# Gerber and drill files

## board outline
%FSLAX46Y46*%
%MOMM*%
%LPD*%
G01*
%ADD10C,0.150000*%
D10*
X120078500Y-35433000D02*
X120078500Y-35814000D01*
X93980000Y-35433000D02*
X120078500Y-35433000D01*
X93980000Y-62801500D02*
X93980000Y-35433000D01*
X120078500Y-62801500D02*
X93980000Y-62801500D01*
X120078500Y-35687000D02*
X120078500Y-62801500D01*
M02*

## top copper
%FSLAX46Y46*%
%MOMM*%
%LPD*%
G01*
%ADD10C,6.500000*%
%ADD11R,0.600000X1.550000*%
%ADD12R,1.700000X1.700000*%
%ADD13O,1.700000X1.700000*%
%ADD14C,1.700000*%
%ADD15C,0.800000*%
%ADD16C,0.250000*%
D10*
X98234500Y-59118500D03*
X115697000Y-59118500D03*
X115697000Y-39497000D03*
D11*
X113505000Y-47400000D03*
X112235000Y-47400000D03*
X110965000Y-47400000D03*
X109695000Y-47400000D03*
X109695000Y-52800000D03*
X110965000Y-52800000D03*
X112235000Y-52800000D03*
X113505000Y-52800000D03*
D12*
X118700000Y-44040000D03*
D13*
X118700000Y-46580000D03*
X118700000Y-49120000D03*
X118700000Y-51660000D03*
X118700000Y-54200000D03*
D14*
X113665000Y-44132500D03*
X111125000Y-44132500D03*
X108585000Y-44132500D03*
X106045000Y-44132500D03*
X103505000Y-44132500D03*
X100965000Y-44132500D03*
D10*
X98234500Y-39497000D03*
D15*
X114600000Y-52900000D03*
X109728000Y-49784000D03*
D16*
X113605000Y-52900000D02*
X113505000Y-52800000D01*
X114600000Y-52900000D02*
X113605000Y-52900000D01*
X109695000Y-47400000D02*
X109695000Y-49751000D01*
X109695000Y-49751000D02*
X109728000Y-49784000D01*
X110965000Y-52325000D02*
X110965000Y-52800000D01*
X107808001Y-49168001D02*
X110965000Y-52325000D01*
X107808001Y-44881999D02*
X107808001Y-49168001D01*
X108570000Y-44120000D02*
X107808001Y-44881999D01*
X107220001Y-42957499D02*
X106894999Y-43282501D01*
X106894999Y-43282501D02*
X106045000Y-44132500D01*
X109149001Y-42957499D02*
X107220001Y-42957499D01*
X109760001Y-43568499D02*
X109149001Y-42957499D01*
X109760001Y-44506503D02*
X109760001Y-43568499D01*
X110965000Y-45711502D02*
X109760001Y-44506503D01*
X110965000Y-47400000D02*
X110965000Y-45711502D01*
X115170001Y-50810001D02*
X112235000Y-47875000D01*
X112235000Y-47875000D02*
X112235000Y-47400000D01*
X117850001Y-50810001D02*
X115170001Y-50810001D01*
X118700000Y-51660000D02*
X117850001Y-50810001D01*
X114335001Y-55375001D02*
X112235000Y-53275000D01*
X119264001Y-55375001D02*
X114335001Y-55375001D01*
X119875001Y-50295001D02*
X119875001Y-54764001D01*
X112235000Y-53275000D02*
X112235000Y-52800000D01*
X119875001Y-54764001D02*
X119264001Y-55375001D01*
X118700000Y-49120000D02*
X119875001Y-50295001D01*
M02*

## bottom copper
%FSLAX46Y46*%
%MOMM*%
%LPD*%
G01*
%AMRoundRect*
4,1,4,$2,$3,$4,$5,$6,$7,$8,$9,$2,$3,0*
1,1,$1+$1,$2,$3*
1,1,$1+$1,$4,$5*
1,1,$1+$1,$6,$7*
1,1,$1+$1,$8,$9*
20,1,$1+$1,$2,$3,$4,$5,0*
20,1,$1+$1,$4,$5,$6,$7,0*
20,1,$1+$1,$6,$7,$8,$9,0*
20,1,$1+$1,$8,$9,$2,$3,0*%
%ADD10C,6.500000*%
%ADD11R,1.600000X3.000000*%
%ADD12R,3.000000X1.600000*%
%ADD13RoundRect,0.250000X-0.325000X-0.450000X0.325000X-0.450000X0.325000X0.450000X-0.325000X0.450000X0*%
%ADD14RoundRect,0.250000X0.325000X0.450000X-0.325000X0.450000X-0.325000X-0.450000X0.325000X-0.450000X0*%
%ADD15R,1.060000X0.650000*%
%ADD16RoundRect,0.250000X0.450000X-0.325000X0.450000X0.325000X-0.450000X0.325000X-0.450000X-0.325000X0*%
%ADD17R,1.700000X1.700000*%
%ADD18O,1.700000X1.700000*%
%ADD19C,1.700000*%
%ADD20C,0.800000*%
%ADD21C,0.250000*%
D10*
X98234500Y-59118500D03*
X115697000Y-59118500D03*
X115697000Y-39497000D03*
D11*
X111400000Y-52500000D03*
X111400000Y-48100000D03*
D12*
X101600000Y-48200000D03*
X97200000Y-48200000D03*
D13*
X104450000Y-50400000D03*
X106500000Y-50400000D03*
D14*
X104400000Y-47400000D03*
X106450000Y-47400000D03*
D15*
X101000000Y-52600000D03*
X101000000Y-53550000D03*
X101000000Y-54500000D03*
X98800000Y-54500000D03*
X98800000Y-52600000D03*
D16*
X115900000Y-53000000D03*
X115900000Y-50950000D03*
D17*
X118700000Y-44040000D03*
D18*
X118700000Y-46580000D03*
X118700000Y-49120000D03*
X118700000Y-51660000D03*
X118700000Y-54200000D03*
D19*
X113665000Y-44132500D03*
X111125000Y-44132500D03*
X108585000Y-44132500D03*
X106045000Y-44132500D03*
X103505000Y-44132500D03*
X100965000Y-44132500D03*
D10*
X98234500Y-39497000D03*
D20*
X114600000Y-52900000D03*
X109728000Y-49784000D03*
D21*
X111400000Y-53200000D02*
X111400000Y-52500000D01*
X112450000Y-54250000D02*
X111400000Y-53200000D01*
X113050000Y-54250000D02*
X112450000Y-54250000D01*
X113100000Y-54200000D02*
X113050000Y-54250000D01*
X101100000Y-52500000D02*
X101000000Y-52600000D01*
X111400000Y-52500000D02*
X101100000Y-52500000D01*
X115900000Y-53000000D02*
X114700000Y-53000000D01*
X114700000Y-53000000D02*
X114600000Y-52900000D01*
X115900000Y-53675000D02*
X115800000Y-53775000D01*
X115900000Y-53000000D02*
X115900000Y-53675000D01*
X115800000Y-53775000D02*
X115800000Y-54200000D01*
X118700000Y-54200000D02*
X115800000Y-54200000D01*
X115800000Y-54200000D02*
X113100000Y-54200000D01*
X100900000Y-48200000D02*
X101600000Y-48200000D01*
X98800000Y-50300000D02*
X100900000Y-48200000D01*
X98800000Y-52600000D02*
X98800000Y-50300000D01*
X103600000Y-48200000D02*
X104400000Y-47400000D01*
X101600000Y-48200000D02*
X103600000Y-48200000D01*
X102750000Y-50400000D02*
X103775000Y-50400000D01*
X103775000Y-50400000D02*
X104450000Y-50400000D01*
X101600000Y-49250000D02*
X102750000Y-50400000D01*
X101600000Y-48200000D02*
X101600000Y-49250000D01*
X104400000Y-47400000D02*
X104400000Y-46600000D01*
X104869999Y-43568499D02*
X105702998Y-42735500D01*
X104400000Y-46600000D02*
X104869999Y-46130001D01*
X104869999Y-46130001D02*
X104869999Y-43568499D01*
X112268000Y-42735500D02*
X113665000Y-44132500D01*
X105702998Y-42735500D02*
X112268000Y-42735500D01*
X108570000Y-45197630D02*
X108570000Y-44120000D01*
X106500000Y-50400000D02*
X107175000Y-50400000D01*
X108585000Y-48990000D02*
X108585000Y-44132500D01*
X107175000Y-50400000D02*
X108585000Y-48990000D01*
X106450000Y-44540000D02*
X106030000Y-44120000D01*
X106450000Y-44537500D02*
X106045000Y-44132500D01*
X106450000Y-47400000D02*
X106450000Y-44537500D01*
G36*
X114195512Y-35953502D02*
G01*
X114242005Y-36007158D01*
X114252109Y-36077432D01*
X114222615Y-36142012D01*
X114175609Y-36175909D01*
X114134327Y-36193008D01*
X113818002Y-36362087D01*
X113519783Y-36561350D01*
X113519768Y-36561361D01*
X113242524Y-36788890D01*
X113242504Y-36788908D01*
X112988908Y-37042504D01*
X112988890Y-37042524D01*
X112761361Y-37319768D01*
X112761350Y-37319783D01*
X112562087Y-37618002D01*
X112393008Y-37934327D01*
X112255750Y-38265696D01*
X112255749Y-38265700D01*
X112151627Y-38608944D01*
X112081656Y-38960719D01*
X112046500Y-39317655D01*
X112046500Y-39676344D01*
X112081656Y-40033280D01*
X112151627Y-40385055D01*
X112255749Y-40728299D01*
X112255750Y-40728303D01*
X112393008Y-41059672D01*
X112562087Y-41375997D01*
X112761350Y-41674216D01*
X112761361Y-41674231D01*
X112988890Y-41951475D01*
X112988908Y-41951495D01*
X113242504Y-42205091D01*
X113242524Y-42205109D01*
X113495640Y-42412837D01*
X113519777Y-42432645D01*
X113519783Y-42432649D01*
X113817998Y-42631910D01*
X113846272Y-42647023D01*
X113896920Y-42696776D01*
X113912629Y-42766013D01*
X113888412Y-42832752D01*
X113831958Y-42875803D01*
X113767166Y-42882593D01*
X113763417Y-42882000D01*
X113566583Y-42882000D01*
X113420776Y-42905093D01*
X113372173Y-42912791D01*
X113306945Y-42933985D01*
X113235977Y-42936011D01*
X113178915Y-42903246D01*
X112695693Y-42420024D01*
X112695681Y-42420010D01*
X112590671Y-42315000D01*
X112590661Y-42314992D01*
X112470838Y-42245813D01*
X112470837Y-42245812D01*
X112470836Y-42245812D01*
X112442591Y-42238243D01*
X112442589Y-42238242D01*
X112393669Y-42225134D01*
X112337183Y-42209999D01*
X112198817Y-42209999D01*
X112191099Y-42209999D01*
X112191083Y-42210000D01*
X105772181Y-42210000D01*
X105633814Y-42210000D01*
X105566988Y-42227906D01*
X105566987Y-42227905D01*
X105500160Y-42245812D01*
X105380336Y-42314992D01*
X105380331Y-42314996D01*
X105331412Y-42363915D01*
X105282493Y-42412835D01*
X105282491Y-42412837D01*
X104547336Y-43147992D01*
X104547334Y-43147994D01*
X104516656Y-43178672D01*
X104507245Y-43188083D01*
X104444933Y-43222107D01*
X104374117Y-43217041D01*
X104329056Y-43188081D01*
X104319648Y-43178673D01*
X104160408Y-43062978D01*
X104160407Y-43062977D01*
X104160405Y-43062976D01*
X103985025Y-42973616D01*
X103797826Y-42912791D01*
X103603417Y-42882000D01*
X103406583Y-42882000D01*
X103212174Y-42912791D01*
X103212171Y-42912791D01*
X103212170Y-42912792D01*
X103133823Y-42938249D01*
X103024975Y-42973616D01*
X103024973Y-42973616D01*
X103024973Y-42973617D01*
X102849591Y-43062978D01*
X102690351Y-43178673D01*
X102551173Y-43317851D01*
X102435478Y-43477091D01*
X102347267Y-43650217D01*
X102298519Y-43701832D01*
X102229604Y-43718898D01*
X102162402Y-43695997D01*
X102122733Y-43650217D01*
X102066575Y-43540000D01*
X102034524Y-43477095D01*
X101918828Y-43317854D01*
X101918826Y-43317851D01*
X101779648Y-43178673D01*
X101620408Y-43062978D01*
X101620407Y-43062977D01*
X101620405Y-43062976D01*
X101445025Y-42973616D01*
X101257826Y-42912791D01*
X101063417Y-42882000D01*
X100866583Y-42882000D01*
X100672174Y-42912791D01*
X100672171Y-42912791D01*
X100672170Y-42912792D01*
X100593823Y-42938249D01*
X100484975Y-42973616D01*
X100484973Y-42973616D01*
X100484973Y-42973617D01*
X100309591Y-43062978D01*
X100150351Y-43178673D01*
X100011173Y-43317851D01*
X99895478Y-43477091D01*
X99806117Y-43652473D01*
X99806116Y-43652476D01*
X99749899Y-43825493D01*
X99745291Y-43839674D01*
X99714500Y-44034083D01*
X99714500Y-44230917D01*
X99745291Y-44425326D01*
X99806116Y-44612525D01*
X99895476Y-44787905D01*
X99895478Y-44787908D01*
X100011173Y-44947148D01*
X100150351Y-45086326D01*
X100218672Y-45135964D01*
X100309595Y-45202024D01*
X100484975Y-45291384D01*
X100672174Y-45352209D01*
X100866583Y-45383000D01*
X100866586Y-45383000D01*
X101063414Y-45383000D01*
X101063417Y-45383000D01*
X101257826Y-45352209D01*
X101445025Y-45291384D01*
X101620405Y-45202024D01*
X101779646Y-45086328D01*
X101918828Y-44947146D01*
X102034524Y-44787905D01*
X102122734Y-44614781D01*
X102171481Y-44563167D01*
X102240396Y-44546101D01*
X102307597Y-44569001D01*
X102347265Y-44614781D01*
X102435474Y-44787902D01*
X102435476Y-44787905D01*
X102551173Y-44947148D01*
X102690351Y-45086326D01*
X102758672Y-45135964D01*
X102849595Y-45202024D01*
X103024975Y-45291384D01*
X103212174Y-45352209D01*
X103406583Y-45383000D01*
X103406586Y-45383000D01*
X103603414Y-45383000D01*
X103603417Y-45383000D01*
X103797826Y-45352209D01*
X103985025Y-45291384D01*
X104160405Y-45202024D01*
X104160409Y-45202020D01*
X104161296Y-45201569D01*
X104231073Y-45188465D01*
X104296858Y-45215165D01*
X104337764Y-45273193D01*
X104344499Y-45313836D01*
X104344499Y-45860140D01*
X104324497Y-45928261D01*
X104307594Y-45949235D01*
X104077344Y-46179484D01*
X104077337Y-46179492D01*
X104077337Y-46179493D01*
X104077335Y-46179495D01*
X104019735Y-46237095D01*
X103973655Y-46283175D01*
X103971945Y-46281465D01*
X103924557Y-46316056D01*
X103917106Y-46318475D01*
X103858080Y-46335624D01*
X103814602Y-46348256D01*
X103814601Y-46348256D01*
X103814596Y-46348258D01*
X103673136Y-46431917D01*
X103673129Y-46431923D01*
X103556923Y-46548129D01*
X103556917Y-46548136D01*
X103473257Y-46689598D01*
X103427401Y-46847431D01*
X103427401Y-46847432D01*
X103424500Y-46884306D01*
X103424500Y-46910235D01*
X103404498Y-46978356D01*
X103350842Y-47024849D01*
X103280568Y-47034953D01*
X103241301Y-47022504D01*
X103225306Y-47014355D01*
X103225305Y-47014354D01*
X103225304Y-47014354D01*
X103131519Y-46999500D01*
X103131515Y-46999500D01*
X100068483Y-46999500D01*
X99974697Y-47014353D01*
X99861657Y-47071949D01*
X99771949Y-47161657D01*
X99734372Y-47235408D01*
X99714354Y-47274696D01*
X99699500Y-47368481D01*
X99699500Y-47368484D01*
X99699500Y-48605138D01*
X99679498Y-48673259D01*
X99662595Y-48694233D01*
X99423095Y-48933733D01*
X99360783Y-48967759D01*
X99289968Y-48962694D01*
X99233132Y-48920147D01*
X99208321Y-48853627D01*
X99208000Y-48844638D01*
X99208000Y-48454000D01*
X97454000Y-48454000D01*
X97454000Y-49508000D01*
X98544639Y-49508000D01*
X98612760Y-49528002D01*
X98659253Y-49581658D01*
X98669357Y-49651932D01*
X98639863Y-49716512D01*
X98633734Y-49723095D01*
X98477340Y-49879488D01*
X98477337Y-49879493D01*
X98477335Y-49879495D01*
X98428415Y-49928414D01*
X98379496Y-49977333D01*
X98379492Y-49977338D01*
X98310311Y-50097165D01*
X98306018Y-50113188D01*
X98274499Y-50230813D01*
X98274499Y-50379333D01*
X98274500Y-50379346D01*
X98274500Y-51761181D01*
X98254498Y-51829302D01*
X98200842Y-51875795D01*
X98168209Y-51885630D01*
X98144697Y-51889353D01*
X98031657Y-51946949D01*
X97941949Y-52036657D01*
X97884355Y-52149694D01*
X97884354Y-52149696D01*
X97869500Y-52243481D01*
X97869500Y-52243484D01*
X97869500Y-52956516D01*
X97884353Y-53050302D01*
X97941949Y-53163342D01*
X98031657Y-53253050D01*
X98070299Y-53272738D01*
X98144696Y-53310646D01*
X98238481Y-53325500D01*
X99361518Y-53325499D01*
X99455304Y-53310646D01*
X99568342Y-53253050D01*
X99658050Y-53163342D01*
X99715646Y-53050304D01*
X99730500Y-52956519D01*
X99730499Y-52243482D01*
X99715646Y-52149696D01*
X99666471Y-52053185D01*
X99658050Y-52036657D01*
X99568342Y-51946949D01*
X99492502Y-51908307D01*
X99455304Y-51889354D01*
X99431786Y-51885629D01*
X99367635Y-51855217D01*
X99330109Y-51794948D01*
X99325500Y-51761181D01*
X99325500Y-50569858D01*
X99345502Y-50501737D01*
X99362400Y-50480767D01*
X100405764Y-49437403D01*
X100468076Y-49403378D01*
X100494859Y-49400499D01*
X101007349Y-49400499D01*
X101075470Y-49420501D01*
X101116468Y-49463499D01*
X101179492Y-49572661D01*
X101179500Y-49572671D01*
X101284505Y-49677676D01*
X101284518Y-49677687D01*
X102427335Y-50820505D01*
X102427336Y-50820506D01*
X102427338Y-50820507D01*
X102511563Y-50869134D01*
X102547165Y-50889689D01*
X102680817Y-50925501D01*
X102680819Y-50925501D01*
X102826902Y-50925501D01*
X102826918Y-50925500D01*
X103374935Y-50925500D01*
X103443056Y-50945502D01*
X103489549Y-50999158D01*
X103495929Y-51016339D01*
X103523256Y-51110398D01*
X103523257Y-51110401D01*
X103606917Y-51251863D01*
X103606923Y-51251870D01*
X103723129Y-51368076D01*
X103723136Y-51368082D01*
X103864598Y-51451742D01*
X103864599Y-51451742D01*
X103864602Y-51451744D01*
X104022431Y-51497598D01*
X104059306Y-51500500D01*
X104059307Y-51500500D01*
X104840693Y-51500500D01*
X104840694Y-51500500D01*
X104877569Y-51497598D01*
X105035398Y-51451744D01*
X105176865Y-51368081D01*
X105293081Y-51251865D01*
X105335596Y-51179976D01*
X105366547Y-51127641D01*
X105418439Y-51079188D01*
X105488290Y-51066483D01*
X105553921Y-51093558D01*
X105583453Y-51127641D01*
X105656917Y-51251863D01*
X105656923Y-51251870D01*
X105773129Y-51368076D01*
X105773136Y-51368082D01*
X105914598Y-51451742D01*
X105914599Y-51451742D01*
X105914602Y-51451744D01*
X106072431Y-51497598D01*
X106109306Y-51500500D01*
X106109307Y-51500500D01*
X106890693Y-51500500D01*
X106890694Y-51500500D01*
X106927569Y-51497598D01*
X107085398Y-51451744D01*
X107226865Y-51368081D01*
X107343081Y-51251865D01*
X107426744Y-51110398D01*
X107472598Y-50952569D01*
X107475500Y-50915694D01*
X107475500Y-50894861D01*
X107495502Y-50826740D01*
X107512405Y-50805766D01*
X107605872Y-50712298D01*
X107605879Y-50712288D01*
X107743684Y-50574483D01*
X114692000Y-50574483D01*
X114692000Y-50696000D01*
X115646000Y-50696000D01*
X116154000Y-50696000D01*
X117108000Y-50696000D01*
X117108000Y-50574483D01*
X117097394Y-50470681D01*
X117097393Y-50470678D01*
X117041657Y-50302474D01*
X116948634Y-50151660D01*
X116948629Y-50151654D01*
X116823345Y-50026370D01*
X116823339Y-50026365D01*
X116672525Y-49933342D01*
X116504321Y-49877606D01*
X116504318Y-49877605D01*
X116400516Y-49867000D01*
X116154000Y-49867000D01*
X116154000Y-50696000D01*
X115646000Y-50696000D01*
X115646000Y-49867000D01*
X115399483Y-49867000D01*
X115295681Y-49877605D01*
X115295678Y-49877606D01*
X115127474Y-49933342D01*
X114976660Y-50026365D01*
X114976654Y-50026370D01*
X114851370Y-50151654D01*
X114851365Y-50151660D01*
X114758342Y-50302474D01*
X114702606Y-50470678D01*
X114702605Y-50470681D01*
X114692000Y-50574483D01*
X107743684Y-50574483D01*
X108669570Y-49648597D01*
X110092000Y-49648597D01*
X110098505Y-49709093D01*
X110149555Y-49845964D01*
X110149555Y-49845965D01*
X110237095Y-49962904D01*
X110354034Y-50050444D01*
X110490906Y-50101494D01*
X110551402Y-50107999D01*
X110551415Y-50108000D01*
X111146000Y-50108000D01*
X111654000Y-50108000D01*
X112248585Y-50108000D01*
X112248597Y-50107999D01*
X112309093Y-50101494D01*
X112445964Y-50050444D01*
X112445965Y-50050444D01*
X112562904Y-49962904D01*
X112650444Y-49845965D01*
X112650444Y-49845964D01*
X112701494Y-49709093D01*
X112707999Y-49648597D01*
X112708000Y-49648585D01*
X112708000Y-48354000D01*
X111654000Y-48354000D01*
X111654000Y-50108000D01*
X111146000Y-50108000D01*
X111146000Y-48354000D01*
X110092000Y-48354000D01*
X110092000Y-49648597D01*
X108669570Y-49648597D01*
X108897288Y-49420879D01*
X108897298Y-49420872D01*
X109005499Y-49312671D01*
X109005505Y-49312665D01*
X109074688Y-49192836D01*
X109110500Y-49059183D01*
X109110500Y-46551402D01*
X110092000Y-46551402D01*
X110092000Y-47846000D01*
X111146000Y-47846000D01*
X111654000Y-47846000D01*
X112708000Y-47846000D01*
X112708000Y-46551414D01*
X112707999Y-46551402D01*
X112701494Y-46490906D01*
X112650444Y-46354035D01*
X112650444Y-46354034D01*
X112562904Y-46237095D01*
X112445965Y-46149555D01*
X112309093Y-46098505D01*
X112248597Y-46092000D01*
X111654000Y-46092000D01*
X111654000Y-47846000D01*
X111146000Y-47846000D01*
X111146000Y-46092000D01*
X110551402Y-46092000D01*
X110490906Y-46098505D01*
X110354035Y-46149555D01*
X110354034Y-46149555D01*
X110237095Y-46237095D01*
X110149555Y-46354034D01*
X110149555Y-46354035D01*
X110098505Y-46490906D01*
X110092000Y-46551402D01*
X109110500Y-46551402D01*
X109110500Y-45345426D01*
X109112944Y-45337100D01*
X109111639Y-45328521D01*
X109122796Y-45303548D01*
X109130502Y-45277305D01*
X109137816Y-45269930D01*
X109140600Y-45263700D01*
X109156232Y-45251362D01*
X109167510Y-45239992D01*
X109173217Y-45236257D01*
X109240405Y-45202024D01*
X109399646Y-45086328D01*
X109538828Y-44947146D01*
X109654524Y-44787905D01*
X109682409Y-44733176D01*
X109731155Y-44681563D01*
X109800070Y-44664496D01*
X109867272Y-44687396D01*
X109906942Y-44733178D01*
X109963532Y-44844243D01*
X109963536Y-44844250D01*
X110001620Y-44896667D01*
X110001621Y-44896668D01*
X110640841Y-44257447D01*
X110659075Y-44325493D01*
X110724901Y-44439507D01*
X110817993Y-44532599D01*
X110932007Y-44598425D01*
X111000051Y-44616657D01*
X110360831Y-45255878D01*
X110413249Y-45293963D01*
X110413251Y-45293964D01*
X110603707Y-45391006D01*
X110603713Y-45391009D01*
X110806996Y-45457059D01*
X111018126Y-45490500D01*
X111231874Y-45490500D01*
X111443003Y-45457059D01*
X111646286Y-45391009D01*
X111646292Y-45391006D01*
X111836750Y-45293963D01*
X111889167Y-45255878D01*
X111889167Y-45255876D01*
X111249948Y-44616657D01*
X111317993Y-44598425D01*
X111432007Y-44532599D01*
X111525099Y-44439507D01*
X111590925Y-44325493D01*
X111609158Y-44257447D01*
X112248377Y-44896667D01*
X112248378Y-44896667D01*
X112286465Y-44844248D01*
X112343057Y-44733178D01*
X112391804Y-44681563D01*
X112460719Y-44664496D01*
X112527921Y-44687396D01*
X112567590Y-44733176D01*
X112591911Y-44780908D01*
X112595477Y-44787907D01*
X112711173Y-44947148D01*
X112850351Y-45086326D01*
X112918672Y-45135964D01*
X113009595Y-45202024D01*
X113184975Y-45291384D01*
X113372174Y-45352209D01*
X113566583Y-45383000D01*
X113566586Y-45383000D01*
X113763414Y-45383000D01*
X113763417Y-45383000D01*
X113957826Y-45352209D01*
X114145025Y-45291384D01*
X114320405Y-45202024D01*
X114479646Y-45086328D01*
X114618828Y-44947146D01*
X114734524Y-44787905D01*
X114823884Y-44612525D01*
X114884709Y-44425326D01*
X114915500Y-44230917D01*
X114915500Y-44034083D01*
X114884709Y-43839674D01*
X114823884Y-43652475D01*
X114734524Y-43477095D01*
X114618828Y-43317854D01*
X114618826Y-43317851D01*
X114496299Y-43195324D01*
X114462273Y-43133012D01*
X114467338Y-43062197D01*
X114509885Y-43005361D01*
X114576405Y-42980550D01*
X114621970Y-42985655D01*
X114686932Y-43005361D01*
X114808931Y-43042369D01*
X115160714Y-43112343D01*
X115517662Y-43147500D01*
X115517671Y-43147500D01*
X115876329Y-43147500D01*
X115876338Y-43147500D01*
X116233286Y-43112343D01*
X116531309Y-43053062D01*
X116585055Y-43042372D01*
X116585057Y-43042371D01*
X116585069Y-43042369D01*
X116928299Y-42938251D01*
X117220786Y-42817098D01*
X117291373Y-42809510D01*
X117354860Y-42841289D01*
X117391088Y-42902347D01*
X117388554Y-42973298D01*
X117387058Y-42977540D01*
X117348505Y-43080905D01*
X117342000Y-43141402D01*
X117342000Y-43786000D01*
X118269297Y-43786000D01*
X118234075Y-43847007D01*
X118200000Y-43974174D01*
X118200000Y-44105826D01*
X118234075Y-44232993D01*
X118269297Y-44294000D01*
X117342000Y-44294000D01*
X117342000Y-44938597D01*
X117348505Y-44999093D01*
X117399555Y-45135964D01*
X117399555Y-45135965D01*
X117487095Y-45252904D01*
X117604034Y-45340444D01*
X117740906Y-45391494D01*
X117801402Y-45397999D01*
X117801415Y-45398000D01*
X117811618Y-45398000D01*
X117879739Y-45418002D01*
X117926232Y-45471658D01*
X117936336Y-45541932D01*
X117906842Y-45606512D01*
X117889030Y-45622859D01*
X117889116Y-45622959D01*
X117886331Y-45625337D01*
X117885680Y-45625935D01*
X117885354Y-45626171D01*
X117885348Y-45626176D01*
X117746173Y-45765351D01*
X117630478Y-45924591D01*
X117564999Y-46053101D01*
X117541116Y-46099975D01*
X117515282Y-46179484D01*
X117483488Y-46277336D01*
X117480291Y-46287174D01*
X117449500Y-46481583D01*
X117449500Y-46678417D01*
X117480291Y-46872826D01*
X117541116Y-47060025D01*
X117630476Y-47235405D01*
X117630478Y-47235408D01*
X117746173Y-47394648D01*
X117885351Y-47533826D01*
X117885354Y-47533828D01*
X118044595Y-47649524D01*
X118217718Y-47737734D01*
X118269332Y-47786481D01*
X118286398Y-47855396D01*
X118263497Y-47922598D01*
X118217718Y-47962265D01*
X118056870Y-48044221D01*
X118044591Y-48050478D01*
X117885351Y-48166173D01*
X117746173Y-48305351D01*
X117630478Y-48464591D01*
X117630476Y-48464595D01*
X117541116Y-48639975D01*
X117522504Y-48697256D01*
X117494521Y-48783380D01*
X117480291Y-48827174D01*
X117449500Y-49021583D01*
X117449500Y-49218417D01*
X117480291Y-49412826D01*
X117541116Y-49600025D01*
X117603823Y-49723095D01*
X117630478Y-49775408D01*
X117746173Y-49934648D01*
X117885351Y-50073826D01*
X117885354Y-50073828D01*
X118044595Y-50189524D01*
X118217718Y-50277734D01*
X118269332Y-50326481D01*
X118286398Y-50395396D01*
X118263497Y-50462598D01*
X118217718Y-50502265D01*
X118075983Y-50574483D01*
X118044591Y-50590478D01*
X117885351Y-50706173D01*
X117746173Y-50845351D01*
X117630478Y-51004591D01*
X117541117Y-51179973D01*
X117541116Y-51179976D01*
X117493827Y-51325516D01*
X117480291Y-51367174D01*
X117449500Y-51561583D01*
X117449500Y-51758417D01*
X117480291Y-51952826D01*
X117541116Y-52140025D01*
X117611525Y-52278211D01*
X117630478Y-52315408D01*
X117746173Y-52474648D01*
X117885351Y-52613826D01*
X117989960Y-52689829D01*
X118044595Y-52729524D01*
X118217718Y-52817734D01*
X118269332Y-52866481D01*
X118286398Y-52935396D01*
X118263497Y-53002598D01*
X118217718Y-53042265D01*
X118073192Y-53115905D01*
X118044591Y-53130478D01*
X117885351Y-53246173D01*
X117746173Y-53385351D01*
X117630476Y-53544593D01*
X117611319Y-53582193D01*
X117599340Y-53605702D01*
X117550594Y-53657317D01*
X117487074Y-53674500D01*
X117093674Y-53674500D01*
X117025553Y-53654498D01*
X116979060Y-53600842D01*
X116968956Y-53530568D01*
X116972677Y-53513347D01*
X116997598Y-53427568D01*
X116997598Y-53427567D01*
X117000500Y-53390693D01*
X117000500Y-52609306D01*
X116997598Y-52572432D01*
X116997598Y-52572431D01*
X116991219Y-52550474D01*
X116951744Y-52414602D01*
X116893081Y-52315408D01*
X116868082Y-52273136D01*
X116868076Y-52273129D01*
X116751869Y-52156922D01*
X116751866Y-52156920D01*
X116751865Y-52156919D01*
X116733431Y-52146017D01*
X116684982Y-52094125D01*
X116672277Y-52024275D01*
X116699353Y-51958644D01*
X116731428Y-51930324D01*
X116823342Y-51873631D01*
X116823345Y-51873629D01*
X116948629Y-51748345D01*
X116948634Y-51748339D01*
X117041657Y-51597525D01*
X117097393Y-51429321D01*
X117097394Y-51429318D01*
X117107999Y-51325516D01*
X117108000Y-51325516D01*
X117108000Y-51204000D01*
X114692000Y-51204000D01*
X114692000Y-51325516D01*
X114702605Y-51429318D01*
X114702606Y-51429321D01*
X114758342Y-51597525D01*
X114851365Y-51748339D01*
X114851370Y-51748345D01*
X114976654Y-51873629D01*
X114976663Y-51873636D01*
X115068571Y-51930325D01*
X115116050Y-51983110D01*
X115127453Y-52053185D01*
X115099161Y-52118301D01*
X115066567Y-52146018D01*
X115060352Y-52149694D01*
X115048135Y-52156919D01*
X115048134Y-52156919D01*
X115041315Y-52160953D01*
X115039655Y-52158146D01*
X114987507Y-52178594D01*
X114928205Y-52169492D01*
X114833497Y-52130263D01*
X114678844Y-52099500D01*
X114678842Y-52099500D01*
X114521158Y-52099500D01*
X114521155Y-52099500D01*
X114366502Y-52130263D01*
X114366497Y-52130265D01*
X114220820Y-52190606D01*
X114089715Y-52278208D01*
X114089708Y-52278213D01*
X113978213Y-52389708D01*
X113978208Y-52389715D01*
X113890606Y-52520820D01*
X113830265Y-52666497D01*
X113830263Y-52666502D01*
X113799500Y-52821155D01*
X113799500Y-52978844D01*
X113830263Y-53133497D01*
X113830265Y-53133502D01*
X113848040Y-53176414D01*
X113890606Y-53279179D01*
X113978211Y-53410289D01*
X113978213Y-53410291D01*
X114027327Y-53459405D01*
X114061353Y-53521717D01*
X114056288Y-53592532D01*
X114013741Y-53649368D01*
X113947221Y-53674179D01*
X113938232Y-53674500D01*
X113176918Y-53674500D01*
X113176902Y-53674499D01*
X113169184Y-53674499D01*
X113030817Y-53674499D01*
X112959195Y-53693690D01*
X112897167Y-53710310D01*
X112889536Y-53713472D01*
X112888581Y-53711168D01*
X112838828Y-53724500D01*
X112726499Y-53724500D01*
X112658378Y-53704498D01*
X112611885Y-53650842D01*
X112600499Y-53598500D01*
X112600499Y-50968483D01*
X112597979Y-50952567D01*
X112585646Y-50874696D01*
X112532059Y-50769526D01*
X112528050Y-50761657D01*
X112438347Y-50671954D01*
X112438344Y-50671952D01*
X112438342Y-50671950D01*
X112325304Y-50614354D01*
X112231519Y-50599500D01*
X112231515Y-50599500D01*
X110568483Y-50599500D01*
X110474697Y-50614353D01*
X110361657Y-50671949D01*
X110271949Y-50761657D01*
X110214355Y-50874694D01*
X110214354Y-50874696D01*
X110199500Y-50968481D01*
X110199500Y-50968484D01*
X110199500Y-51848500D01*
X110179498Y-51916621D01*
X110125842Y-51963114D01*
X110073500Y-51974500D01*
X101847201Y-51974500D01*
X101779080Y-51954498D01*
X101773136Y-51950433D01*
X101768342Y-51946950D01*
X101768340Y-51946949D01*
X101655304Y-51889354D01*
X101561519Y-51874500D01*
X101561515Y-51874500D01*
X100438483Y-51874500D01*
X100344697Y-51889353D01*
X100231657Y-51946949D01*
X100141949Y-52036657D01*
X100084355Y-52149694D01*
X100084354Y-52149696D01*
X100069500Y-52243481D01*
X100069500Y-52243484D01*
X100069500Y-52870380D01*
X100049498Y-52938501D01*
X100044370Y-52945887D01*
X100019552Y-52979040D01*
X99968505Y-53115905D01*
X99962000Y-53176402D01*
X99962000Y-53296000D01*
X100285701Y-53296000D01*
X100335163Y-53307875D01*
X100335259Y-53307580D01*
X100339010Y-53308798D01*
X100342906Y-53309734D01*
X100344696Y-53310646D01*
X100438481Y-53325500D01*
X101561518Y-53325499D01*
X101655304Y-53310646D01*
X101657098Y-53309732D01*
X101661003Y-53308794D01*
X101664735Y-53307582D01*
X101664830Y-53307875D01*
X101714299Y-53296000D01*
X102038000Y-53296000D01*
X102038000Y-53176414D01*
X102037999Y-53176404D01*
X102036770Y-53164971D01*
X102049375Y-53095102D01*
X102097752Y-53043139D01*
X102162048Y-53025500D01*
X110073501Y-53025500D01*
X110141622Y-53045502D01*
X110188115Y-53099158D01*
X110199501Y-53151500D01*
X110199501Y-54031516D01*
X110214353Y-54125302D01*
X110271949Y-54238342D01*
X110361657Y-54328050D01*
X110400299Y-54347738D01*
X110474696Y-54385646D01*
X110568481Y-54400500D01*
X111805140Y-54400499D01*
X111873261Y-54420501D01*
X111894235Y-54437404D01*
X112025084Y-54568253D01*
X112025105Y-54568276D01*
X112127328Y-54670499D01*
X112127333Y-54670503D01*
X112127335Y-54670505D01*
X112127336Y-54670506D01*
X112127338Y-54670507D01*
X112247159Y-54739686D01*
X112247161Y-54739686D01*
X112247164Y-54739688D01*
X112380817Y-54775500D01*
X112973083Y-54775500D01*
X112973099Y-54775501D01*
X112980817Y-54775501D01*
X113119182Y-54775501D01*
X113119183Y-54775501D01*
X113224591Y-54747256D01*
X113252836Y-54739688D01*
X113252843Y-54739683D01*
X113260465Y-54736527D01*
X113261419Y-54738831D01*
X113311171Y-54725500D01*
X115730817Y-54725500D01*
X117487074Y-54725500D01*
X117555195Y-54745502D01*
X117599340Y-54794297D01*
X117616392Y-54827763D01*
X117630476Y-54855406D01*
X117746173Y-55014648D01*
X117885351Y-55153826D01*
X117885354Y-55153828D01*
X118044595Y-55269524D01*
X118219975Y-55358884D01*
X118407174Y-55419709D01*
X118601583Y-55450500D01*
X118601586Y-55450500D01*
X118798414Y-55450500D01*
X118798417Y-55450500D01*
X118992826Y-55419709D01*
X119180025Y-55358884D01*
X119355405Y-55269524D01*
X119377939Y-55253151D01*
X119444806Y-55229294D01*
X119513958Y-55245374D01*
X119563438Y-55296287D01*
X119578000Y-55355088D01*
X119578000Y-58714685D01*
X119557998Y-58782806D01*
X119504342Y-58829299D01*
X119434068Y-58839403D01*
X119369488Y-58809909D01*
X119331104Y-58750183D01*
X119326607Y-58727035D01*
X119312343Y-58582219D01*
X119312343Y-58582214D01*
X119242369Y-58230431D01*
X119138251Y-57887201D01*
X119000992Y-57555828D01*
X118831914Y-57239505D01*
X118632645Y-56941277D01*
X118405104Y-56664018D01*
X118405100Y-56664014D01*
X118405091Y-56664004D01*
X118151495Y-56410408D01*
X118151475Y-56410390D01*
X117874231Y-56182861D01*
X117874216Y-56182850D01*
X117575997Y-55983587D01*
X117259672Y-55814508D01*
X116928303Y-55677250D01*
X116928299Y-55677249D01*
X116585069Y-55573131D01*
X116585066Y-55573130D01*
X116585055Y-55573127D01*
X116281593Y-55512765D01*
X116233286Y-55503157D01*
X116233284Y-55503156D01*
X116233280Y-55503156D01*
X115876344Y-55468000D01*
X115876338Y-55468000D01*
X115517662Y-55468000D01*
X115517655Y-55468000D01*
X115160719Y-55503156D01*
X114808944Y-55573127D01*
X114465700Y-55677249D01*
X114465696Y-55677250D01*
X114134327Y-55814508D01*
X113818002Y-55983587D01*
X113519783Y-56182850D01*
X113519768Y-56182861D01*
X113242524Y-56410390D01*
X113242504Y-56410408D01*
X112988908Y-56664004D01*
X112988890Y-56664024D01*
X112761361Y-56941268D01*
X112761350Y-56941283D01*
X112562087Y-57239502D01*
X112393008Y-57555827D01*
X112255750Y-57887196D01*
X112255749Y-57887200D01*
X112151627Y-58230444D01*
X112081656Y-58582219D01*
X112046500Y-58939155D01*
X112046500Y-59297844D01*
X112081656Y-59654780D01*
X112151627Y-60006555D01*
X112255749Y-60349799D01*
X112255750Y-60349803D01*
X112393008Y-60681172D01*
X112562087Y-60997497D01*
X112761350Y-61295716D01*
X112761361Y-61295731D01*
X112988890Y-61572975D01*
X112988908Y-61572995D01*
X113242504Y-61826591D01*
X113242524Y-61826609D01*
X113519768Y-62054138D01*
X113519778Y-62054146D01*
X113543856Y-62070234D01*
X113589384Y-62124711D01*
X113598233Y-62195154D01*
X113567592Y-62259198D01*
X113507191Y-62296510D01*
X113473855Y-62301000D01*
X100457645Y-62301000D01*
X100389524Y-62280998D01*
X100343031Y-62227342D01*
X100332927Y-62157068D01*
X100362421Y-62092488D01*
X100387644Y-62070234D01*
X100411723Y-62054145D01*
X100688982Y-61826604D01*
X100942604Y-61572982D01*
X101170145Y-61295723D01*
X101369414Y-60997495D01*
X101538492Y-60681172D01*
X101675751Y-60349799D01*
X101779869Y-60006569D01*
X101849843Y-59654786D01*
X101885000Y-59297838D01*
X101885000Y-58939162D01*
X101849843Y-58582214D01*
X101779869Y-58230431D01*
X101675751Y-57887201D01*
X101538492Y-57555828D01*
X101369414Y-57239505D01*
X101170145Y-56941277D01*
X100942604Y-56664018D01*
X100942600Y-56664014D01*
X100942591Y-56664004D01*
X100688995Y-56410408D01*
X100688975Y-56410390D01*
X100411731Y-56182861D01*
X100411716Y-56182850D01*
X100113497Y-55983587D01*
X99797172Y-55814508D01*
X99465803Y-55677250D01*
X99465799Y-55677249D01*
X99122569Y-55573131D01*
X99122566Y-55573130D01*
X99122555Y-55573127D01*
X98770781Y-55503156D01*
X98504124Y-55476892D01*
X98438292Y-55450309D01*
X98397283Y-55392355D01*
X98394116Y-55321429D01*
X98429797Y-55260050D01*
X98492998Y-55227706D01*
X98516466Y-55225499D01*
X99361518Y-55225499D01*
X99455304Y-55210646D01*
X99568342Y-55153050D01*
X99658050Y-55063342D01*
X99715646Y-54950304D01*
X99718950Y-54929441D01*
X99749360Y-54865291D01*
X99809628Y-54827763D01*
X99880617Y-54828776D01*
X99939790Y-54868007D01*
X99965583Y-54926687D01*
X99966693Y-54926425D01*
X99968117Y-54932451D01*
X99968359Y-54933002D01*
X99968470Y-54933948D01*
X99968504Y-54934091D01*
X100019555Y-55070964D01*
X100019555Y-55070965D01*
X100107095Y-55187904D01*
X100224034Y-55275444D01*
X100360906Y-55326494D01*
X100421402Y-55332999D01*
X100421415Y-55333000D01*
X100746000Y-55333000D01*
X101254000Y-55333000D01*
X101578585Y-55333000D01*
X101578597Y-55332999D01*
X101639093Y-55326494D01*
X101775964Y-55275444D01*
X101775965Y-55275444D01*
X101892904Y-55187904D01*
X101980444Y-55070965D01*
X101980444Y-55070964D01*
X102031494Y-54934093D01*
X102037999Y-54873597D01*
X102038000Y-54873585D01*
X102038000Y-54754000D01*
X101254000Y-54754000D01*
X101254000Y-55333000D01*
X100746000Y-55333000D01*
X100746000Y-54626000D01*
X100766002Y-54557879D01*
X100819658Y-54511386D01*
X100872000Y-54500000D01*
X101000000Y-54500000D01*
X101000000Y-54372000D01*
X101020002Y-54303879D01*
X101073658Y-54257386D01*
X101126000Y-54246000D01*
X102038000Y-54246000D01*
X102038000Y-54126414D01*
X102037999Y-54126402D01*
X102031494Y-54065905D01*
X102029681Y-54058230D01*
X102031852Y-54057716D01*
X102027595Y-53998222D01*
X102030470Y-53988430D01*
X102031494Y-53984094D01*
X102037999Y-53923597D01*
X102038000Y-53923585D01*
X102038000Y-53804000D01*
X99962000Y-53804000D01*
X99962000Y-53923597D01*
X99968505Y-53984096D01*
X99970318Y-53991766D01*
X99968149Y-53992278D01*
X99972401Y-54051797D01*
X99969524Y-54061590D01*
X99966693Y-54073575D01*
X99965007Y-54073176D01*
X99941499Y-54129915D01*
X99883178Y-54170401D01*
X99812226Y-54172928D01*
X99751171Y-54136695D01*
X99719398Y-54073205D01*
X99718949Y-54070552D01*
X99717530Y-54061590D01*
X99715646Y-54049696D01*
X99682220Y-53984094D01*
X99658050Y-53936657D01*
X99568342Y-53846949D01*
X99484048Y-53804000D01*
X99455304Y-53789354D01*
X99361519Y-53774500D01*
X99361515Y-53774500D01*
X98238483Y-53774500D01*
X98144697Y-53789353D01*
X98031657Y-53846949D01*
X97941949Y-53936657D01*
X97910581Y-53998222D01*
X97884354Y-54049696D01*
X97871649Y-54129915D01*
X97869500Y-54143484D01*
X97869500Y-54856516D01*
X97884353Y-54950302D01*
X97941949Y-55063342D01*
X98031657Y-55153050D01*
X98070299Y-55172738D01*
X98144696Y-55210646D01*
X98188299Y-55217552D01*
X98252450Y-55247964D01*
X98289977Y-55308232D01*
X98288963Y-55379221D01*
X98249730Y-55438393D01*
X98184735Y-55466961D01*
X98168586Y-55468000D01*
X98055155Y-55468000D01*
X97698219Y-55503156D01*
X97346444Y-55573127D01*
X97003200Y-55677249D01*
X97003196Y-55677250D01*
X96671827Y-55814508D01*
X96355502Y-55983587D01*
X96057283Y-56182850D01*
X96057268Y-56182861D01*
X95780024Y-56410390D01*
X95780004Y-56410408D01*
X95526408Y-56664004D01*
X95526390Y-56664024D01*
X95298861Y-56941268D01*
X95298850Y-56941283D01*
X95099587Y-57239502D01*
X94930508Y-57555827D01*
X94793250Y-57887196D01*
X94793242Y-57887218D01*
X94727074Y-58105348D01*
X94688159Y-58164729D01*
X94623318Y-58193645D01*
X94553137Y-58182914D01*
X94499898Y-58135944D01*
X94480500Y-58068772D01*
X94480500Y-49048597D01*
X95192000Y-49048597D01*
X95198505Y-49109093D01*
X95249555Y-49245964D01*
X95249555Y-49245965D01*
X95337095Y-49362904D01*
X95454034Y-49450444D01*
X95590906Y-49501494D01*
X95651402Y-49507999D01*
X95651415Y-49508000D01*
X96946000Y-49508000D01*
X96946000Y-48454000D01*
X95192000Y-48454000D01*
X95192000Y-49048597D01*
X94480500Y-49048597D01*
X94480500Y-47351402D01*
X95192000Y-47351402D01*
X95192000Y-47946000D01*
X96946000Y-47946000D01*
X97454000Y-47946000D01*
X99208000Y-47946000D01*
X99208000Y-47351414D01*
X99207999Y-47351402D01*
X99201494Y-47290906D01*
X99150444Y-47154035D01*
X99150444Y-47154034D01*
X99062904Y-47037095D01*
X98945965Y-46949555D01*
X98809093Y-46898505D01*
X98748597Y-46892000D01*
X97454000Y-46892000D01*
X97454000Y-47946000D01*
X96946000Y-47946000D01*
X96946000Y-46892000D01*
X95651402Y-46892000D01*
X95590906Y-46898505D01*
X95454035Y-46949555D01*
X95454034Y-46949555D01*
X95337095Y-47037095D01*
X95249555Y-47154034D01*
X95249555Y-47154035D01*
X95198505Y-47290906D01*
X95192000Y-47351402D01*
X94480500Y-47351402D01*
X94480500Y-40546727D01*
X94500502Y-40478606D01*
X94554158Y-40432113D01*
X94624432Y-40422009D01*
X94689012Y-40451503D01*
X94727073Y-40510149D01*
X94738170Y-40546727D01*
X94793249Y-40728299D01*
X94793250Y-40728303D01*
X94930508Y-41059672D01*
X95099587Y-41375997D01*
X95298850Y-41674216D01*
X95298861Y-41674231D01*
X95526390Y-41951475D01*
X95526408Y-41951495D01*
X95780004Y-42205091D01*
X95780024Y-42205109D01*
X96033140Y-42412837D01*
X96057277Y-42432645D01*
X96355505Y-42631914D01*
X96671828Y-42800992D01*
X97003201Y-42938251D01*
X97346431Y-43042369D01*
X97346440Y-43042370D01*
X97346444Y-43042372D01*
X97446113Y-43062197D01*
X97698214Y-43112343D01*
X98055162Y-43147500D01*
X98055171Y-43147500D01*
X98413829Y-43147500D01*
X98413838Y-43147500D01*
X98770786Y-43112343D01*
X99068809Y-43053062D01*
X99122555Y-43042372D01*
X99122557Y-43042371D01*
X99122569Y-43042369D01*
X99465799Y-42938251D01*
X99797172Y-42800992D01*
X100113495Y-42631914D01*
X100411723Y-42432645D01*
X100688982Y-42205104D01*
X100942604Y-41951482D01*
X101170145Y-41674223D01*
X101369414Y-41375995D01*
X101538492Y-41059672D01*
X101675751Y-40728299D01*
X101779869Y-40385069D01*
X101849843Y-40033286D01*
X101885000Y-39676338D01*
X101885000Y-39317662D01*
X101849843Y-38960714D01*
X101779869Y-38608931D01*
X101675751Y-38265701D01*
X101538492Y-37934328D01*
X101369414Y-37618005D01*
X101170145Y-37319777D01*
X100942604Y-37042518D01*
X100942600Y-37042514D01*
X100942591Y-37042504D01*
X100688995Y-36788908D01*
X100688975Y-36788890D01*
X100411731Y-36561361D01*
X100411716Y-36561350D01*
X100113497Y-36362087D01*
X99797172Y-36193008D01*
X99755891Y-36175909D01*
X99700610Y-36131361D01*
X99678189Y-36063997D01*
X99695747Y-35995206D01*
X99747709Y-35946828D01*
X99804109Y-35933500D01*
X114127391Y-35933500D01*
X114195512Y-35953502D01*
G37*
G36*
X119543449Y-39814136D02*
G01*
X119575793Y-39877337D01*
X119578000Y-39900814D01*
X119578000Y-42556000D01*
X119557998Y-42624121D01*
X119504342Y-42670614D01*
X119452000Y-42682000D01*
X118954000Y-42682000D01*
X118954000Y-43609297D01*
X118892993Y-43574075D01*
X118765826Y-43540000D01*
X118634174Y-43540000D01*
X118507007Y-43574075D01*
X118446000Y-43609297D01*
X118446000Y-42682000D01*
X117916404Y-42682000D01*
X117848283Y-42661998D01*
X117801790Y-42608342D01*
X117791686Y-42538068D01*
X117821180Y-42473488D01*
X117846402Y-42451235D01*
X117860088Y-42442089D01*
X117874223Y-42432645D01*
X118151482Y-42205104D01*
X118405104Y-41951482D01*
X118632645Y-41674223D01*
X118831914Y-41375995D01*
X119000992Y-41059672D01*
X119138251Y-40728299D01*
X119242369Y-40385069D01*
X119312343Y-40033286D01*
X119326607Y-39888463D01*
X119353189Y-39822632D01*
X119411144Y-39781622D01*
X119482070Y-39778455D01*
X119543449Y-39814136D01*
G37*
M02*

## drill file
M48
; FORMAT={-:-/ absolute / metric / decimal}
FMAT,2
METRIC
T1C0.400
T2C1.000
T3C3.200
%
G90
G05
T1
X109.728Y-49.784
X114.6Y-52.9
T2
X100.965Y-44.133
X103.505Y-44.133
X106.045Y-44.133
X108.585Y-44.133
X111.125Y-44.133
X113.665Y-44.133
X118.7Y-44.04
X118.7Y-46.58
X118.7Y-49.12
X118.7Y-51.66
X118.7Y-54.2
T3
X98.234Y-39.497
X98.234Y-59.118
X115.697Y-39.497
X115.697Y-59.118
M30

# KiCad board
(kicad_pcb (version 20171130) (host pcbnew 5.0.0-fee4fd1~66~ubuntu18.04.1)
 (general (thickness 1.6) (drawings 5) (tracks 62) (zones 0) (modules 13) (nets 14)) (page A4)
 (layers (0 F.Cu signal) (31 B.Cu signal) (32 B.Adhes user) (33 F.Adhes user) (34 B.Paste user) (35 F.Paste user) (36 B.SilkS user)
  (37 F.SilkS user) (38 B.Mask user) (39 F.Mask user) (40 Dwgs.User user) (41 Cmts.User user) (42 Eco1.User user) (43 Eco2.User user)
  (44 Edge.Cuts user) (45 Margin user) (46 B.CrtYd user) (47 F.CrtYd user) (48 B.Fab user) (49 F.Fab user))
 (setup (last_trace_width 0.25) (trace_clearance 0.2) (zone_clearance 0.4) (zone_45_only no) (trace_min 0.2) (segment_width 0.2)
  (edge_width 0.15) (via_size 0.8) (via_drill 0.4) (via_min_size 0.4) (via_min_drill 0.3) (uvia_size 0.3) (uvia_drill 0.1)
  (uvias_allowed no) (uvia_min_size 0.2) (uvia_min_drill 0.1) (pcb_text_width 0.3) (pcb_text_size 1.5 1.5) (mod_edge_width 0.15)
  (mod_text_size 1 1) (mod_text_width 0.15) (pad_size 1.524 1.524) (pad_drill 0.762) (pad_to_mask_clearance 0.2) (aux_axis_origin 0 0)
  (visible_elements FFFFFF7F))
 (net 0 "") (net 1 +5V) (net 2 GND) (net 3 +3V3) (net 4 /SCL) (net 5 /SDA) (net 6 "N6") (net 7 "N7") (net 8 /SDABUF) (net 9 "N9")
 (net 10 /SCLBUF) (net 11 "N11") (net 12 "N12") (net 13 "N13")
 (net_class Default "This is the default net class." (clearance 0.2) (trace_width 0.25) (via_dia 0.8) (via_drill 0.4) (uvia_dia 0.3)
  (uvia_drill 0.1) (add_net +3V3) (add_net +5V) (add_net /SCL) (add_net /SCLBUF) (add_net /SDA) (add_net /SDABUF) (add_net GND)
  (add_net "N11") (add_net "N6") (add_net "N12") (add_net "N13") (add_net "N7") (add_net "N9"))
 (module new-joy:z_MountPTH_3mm (layer F.Cu) (at 98.2345 59.1185)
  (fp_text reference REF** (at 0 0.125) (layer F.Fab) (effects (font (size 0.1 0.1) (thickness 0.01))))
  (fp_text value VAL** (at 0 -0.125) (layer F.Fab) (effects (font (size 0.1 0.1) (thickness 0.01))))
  (pad 1 thru_hole circle (at 0 0) (size 6.5 6.5) (drill 3.2) (layers *.Cu *.Mask)))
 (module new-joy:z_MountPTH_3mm (layer F.Cu) (at 115.697 59.1185)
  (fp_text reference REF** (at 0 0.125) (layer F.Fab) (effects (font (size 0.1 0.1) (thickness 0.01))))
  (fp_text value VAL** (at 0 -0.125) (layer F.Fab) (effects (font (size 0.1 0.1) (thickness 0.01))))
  (pad 1 thru_hole circle (at 0 0) (size 6.5 6.5) (drill 3.2) (layers *.Cu *.Mask)))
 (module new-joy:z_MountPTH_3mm (layer F.Cu) (at 115.697 39.497)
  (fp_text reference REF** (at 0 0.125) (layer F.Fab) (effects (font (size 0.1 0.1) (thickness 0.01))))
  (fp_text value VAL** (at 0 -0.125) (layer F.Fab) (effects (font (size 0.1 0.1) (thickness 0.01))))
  (pad 1 thru_hole circle (at 0 0) (size 6.5 6.5) (drill 3.2) (layers *.Cu *.Mask)))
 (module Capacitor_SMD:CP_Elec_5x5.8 (layer B.Cu) (at 111.4 50.3 90)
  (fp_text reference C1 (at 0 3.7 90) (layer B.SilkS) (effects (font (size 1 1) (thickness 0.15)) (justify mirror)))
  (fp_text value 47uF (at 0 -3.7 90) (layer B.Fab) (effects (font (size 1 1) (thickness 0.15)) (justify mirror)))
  (pad 1 smd rect (at -2.2 0 90) (size 3 1.6) (layers B.Cu B.Paste B.Mask) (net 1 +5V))
  (pad 2 smd rect (at 2.2 0 90) (size 3 1.6) (layers B.Cu B.Paste B.Mask) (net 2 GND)))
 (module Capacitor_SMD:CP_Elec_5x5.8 (layer B.Cu) (at 99.4 48.2 180)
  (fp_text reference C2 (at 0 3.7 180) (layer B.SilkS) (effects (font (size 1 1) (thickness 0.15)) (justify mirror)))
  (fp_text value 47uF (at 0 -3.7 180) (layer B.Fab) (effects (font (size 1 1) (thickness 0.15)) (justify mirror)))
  (pad 1 smd rect (at -2.2 0 180) (size 3 1.6) (layers B.Cu B.Paste B.Mask) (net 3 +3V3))
  (pad 2 smd rect (at 2.2 0 180) (size 3 1.6) (layers B.Cu B.Paste B.Mask) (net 2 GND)))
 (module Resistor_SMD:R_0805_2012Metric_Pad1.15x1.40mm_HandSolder (layer B.Cu) (at 105.475 50.4)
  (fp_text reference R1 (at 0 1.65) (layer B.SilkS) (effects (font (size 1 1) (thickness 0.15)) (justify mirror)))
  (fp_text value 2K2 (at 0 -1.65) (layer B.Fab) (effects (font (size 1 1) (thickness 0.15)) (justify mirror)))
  (pad 1 smd roundrect (at -1.025 0) (size 1.15 1.4) (layers B.Cu B.Paste B.Mask) (roundrect_rratio 0.217391) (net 3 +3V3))
  (pad 2 smd roundrect (at 1.025 0) (size 1.15 1.4) (layers B.Cu B.Paste B.Mask) (roundrect_rratio 0.217391) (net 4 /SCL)))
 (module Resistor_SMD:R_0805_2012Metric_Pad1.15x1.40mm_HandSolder (layer B.Cu) (at 105.425 47.4 180)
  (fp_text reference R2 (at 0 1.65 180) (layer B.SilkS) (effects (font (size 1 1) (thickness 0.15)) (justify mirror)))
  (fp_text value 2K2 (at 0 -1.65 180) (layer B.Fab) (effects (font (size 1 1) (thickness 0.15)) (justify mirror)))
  (pad 2 smd roundrect (at 1.025 0 180) (size 1.15 1.4) (layers B.Cu B.Paste B.Mask) (roundrect_rratio 0.217391) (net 3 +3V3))
  (pad 1 smd roundrect (at -1.025 0 180) (size 1.15 1.4) (layers B.Cu B.Paste B.Mask) (roundrect_rratio 0.217391) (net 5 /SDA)))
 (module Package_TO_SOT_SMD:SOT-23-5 (layer B.Cu) (at 99.9 53.55 180)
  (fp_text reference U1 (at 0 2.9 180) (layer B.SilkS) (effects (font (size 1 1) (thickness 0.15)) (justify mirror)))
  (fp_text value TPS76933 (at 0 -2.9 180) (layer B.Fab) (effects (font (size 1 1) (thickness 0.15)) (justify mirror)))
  (pad 1 smd rect (at -1.1 0.95 180) (size 1.06 0.65) (layers B.Cu B.Paste B.Mask) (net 1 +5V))
  (pad 2 smd rect (at -1.1 0 180) (size 1.06 0.65) (layers B.Cu B.Paste B.Mask) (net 2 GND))
  (pad 3 smd rect (at -1.1 -0.95 180) (size 1.06 0.65) (layers B.Cu B.Paste B.Mask) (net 2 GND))
  (pad 4 smd rect (at 1.1 -0.95 180) (size 1.06 0.65) (layers B.Cu B.Paste B.Mask) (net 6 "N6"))
  (pad 5 smd rect (at 1.1 0.95 180) (size 1.06 0.65) (layers B.Cu B.Paste B.Mask) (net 3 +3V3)))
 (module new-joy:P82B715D (layer F.Cu) (at 111.6 50.1 270)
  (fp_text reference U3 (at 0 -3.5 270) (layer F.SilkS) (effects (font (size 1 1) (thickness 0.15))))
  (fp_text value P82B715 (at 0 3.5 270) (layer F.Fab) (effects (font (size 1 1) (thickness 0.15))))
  (pad 1 smd rect (at -2.7 -1.905 270) (size 1.55 0.6) (layers F.Cu F.Paste F.Mask) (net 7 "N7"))
  (pad 2 smd rect (at -2.7 -0.635 270) (size 1.55 0.6) (layers F.Cu F.Paste F.Mask) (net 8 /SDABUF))
  (pad 3 smd rect (at -2.7 0.635 270) (size 1.55 0.6) (layers F.Cu F.Paste F.Mask) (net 5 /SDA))
  (pad 4 smd rect (at -2.7 1.905 270) (size 1.55 0.6) (layers F.Cu F.Paste F.Mask) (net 2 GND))
  (pad 5 smd rect (at 2.7 1.905 270) (size 1.55 0.6) (layers F.Cu F.Paste F.Mask) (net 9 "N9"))
  (pad 6 smd rect (at 2.7 0.635 270) (size 1.55 0.6) (layers F.Cu F.Paste F.Mask) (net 4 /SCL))
  (pad 7 smd rect (at 2.7 -0.635 270) (size 1.55 0.6) (layers F.Cu F.Paste F.Mask) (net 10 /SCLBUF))
  (pad 8 smd rect (at 2.7 -1.905 270) (size 1.55 0.6) (layers F.Cu F.Paste F.Mask) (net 1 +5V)))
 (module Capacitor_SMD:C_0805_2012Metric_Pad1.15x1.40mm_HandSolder (layer B.Cu) (at 115.9 51.975 90)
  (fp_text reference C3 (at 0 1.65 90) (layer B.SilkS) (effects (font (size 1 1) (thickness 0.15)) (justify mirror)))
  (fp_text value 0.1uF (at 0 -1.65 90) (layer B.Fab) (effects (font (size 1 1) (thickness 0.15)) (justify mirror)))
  (pad 1 smd roundrect (at -1.025 0 90) (size 1.15 1.4) (layers B.Cu B.Paste B.Mask) (roundrect_rratio 0.217391) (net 1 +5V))
  (pad 2 smd roundrect (at 1.025 0 90) (size 1.15 1.4) (layers B.Cu B.Paste B.Mask) (roundrect_rratio 0.217391) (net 2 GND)))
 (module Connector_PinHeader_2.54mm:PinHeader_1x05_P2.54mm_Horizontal (layer F.Cu) (at 118.7 44.04)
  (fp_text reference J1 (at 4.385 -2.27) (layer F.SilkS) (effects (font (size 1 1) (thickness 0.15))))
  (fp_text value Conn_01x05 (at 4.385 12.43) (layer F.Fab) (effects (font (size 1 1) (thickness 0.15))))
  (pad 1 thru_hole rect (at 0 0) (size 1.7 1.7) (drill 1) (layers *.Cu *.Mask) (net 2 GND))
  (pad 2 thru_hole oval (at 0 2.54) (size 1.7 1.7) (drill 1) (layers *.Cu *.Mask) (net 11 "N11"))
  (pad 3 thru_hole oval (at 0 5.08) (size 1.7 1.7) (drill 1) (layers *.Cu *.Mask) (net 10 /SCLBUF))
  (pad 4 thru_hole oval (at 0 7.62) (size 1.7 1.7) (drill 1) (layers *.Cu *.Mask) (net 8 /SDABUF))
  (pad 5 thru_hole oval (at 0 10.16) (size 1.7 1.7) (drill 1) (layers *.Cu *.Mask) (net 1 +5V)))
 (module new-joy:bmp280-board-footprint (layer F.Cu) (at 107.315 49.2125 270)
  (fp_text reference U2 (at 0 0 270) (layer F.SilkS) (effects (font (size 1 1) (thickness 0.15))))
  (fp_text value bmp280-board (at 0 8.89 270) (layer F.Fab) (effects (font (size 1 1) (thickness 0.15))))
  (pad 1 thru_hole circle (at -5.08 -6.35 270) (size 1.7 1.7) (drill 1) (layers *.Cu *.Mask) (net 3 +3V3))
  (pad 2 thru_hole circle (at -5.08 -3.81 270) (size 1.7 1.7) (drill 1) (layers *.Cu *.Mask) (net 2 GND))
  (pad 3 thru_hole circle (at -5.08 -1.27 270) (size 1.7 1.7) (drill 1) (layers *.Cu *.Mask) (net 4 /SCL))
  (pad 4 thru_hole circle (at -5.08 1.27 270) (size 1.7 1.7) (drill 1) (layers *.Cu *.Mask) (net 5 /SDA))
  (pad 5 thru_hole circle (at -5.08 3.81 270) (size 1.7 1.7) (drill 1) (layers *.Cu *.Mask) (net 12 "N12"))
  (pad 6 thru_hole circle (at -5.08 6.35 270) (size 1.7 1.7) (drill 1) (layers *.Cu *.Mask) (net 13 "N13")))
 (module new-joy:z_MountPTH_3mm (layer F.Cu) (at 98.2345 39.497)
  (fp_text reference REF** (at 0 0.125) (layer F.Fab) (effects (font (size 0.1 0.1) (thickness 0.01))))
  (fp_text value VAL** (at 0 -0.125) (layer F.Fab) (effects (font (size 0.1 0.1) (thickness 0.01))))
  (pad 1 thru_hole circle (at 0 0) (size 6.5 6.5) (drill 3.2) (layers *.Cu *.Mask)))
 (gr_line (start 120.0785 35.433) (end 120.0785 35.814) (layer Edge.Cuts) (width 0.15))
 (gr_line (start 93.98 35.433) (end 120.0785 35.433) (layer Edge.Cuts) (width 0.15))
 (gr_line (start 93.98 62.8015) (end 93.98 35.433) (layer Edge.Cuts) (width 0.15))
 (gr_line (start 120.0785 62.8015) (end 93.98 62.8015) (layer Edge.Cuts) (width 0.15))
 (gr_line (start 120.0785 35.687) (end 120.0785 62.8015) (layer Edge.Cuts) (width 0.15))
 (segment (start 111.4 53.2) (end 111.4 52.5) (width 0.25) (layer B.Cu) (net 1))
 (segment (start 112.45 54.25) (end 111.4 53.2) (width 0.25) (layer B.Cu) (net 1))
 (segment (start 113.05 54.25) (end 112.45 54.25) (width 0.25) (layer B.Cu) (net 1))
 (segment (start 113.1 54.2) (end 113.05 54.25) (width 0.25) (layer B.Cu) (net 1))
 (segment (start 101.1 52.5) (end 101 52.6) (width 0.25) (layer B.Cu) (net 1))
 (segment (start 111.4 52.5) (end 101.1 52.5) (width 0.25) (layer B.Cu) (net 1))
 (via (at 114.6 52.9) (size 0.8) (drill 0.4) (layers F.Cu B.Cu) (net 1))
 (segment (start 115.9 53) (end 114.7 53) (width 0.25) (layer B.Cu) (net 1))
 (segment (start 114.7 53) (end 114.6 52.9) (width 0.25) (layer B.Cu) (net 1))
 (segment (start 113.605 52.9) (end 113.505 52.8) (width 0.25) (layer F.Cu) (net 1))
 (segment (start 114.6 52.9) (end 113.605 52.9) (width 0.25) (layer F.Cu) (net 1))
 (segment (start 115.9 53.675) (end 115.8 53.775) (width 0.25) (layer B.Cu) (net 1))
 (segment (start 115.9 53) (end 115.9 53.675) (width 0.25) (layer B.Cu) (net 1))
 (segment (start 115.8 53.775) (end 115.8 54.2) (width 0.25) (layer B.Cu) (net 1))
 (segment (start 118.7 54.2) (end 115.8 54.2) (width 0.25) (layer B.Cu) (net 1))
 (segment (start 115.8 54.2) (end 113.1 54.2) (width 0.25) (layer B.Cu) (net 1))
 (via (at 109.728 49.784) (size 0.8) (drill 0.4) (layers F.Cu B.Cu) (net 2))
 (segment (start 109.695 47.4) (end 109.695 49.751) (width 0.25) (layer F.Cu) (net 2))
 (segment (start 109.695 49.751) (end 109.728 49.784) (width 0.25) (layer F.Cu) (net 2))
 (segment (start 100.9 48.2) (end 101.6 48.2) (width 0.25) (layer B.Cu) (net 3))
 (segment (start 98.8 50.3) (end 100.9 48.2) (width 0.25) (layer B.Cu) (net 3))
 (segment (start 98.8 52.6) (end 98.8 50.3) (width 0.25) (layer B.Cu) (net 3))
 (segment (start 103.6 48.2) (end 104.4 47.4) (width 0.25) (layer B.Cu) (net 3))
 (segment (start 101.6 48.2) (end 103.6 48.2) (width 0.25) (layer B.Cu) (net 3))
 (segment (start 102.75 50.4) (end 103.775 50.4) (width 0.25) (layer B.Cu) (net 3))
 (segment (start 103.775 50.4) (end 104.45 50.4) (width 0.25) (layer B.Cu) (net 3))
 (segment (start 101.6 49.25) (end 102.75 50.4) (width 0.25) (layer B.Cu) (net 3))
 (segment (start 101.6 48.2) (end 101.6 49.25) (width 0.25) (layer B.Cu) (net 3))
 (segment (start 104.4 47.4) (end 104.4 46.6) (width 0.25) (layer B.Cu) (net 3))
 (segment (start 104.869999 43.568499) (end 105.702998 42.7355) (width 0.25) (layer B.Cu) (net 3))
 (segment (start 104.4 46.6) (end 104.869999 46.130001) (width 0.25) (layer B.Cu) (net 3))
 (segment (start 104.869999 46.130001) (end 104.869999 43.568499) (width 0.25) (layer B.Cu) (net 3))
 (segment (start 112.268 42.7355) (end 113.665 44.1325) (width 0.25) (layer B.Cu) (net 3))
 (segment (start 105.702998 42.7355) (end 112.268 42.7355) (width 0.25) (layer B.Cu) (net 3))
 (segment (start 110.965 52.325) (end 110.965 52.8) (width 0.25) (layer F.Cu) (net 4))
 (segment (start 107.808001 49.168001) (end 110.965 52.325) (width 0.25) (layer F.Cu) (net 4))
 (segment (start 107.808001 44.881999) (end 107.808001 49.168001) (width 0.25) (layer F.Cu) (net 4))
 (segment (start 108.57 44.12) (end 107.808001 44.881999) (width 0.25) (layer F.Cu) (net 4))
 (segment (start 108.57 45.19763) (end 108.57 44.12) (width 0.25) (layer B.Cu) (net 4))
 (segment (start 106.5 50.4) (end 107.175 50.4) (width 0.25) (layer B.Cu) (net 4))
 (segment (start 108.585 48.99) (end 108.585 44.1325) (width 0.25) (layer B.Cu) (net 4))
 (segment (start 107.175 50.4) (end 108.585 48.99) (width 0.25) (layer B.Cu) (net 4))
 (segment (start 106.45 44.54) (end 106.03 44.12) (width 0.25) (layer B.Cu) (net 5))
 (segment (start 106.45 44.5375) (end 106.045 44.1325) (width 0.25) (layer B.Cu) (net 5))
 (segment (start 106.45 47.4) (end 106.45 44.5375) (width 0.25) (layer B.Cu) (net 5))
 (segment (start 107.220001 42.957499) (end 106.894999 43.282501) (width 0.25) (layer F.Cu) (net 5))
 (segment (start 106.894999 43.282501) (end 106.045 44.1325) (width 0.25) (layer F.Cu) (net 5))
 (segment (start 109.149001 42.957499) (end 107.220001 42.957499) (width 0.25) (layer F.Cu) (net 5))
 (segment (start 109.760001 43.568499) (end 109.149001 42.957499) (width 0.25) (layer F.Cu) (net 5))
 (segment (start 109.760001 44.506503) (end 109.760001 43.568499) (width 0.25) (layer F.Cu) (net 5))
 (segment (start 110.965 45.711502) (end 109.760001 44.506503) (width 0.25) (layer F.Cu) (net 5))
 (segment (start 110.965 47.4) (end 110.965 45.711502) (width 0.25) (layer F.Cu) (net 5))
 (segment (start 115.170001 50.810001) (end 112.235 47.875) (width 0.25) (layer F.Cu) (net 8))
 (segment (start 112.235 47.875) (end 112.235 47.4) (width 0.25) (layer F.Cu) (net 8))
 (segment (start 117.850001 50.810001) (end 115.170001 50.810001) (width 0.25) (layer F.Cu) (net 8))
 (segment (start 118.7 51.66) (end 117.850001 50.810001) (width 0.25) (layer F.Cu) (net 8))
 (segment (start 114.335001 55.375001) (end 112.235 53.275) (width 0.25) (layer F.Cu) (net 10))
 (segment (start 119.264001 55.375001) (end 114.335001 55.375001) (width 0.25) (layer F.Cu) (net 10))
 (segment (start 119.875001 50.295001) (end 119.875001 54.764001) (width 0.25) (layer F.Cu) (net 10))
 (segment (start 112.235 53.275) (end 112.235 52.8) (width 0.25) (layer F.Cu) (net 10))
 (segment (start 119.875001 54.764001) (end 119.264001 55.375001) (width 0.25) (layer F.Cu) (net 10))
 (segment (start 118.7 49.12) (end 119.875001 50.295001) (width 0.25) (layer F.Cu) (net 10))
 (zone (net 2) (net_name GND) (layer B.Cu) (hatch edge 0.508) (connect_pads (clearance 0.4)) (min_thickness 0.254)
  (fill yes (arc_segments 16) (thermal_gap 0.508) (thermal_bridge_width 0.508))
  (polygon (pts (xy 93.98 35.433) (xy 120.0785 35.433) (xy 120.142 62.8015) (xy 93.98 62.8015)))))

